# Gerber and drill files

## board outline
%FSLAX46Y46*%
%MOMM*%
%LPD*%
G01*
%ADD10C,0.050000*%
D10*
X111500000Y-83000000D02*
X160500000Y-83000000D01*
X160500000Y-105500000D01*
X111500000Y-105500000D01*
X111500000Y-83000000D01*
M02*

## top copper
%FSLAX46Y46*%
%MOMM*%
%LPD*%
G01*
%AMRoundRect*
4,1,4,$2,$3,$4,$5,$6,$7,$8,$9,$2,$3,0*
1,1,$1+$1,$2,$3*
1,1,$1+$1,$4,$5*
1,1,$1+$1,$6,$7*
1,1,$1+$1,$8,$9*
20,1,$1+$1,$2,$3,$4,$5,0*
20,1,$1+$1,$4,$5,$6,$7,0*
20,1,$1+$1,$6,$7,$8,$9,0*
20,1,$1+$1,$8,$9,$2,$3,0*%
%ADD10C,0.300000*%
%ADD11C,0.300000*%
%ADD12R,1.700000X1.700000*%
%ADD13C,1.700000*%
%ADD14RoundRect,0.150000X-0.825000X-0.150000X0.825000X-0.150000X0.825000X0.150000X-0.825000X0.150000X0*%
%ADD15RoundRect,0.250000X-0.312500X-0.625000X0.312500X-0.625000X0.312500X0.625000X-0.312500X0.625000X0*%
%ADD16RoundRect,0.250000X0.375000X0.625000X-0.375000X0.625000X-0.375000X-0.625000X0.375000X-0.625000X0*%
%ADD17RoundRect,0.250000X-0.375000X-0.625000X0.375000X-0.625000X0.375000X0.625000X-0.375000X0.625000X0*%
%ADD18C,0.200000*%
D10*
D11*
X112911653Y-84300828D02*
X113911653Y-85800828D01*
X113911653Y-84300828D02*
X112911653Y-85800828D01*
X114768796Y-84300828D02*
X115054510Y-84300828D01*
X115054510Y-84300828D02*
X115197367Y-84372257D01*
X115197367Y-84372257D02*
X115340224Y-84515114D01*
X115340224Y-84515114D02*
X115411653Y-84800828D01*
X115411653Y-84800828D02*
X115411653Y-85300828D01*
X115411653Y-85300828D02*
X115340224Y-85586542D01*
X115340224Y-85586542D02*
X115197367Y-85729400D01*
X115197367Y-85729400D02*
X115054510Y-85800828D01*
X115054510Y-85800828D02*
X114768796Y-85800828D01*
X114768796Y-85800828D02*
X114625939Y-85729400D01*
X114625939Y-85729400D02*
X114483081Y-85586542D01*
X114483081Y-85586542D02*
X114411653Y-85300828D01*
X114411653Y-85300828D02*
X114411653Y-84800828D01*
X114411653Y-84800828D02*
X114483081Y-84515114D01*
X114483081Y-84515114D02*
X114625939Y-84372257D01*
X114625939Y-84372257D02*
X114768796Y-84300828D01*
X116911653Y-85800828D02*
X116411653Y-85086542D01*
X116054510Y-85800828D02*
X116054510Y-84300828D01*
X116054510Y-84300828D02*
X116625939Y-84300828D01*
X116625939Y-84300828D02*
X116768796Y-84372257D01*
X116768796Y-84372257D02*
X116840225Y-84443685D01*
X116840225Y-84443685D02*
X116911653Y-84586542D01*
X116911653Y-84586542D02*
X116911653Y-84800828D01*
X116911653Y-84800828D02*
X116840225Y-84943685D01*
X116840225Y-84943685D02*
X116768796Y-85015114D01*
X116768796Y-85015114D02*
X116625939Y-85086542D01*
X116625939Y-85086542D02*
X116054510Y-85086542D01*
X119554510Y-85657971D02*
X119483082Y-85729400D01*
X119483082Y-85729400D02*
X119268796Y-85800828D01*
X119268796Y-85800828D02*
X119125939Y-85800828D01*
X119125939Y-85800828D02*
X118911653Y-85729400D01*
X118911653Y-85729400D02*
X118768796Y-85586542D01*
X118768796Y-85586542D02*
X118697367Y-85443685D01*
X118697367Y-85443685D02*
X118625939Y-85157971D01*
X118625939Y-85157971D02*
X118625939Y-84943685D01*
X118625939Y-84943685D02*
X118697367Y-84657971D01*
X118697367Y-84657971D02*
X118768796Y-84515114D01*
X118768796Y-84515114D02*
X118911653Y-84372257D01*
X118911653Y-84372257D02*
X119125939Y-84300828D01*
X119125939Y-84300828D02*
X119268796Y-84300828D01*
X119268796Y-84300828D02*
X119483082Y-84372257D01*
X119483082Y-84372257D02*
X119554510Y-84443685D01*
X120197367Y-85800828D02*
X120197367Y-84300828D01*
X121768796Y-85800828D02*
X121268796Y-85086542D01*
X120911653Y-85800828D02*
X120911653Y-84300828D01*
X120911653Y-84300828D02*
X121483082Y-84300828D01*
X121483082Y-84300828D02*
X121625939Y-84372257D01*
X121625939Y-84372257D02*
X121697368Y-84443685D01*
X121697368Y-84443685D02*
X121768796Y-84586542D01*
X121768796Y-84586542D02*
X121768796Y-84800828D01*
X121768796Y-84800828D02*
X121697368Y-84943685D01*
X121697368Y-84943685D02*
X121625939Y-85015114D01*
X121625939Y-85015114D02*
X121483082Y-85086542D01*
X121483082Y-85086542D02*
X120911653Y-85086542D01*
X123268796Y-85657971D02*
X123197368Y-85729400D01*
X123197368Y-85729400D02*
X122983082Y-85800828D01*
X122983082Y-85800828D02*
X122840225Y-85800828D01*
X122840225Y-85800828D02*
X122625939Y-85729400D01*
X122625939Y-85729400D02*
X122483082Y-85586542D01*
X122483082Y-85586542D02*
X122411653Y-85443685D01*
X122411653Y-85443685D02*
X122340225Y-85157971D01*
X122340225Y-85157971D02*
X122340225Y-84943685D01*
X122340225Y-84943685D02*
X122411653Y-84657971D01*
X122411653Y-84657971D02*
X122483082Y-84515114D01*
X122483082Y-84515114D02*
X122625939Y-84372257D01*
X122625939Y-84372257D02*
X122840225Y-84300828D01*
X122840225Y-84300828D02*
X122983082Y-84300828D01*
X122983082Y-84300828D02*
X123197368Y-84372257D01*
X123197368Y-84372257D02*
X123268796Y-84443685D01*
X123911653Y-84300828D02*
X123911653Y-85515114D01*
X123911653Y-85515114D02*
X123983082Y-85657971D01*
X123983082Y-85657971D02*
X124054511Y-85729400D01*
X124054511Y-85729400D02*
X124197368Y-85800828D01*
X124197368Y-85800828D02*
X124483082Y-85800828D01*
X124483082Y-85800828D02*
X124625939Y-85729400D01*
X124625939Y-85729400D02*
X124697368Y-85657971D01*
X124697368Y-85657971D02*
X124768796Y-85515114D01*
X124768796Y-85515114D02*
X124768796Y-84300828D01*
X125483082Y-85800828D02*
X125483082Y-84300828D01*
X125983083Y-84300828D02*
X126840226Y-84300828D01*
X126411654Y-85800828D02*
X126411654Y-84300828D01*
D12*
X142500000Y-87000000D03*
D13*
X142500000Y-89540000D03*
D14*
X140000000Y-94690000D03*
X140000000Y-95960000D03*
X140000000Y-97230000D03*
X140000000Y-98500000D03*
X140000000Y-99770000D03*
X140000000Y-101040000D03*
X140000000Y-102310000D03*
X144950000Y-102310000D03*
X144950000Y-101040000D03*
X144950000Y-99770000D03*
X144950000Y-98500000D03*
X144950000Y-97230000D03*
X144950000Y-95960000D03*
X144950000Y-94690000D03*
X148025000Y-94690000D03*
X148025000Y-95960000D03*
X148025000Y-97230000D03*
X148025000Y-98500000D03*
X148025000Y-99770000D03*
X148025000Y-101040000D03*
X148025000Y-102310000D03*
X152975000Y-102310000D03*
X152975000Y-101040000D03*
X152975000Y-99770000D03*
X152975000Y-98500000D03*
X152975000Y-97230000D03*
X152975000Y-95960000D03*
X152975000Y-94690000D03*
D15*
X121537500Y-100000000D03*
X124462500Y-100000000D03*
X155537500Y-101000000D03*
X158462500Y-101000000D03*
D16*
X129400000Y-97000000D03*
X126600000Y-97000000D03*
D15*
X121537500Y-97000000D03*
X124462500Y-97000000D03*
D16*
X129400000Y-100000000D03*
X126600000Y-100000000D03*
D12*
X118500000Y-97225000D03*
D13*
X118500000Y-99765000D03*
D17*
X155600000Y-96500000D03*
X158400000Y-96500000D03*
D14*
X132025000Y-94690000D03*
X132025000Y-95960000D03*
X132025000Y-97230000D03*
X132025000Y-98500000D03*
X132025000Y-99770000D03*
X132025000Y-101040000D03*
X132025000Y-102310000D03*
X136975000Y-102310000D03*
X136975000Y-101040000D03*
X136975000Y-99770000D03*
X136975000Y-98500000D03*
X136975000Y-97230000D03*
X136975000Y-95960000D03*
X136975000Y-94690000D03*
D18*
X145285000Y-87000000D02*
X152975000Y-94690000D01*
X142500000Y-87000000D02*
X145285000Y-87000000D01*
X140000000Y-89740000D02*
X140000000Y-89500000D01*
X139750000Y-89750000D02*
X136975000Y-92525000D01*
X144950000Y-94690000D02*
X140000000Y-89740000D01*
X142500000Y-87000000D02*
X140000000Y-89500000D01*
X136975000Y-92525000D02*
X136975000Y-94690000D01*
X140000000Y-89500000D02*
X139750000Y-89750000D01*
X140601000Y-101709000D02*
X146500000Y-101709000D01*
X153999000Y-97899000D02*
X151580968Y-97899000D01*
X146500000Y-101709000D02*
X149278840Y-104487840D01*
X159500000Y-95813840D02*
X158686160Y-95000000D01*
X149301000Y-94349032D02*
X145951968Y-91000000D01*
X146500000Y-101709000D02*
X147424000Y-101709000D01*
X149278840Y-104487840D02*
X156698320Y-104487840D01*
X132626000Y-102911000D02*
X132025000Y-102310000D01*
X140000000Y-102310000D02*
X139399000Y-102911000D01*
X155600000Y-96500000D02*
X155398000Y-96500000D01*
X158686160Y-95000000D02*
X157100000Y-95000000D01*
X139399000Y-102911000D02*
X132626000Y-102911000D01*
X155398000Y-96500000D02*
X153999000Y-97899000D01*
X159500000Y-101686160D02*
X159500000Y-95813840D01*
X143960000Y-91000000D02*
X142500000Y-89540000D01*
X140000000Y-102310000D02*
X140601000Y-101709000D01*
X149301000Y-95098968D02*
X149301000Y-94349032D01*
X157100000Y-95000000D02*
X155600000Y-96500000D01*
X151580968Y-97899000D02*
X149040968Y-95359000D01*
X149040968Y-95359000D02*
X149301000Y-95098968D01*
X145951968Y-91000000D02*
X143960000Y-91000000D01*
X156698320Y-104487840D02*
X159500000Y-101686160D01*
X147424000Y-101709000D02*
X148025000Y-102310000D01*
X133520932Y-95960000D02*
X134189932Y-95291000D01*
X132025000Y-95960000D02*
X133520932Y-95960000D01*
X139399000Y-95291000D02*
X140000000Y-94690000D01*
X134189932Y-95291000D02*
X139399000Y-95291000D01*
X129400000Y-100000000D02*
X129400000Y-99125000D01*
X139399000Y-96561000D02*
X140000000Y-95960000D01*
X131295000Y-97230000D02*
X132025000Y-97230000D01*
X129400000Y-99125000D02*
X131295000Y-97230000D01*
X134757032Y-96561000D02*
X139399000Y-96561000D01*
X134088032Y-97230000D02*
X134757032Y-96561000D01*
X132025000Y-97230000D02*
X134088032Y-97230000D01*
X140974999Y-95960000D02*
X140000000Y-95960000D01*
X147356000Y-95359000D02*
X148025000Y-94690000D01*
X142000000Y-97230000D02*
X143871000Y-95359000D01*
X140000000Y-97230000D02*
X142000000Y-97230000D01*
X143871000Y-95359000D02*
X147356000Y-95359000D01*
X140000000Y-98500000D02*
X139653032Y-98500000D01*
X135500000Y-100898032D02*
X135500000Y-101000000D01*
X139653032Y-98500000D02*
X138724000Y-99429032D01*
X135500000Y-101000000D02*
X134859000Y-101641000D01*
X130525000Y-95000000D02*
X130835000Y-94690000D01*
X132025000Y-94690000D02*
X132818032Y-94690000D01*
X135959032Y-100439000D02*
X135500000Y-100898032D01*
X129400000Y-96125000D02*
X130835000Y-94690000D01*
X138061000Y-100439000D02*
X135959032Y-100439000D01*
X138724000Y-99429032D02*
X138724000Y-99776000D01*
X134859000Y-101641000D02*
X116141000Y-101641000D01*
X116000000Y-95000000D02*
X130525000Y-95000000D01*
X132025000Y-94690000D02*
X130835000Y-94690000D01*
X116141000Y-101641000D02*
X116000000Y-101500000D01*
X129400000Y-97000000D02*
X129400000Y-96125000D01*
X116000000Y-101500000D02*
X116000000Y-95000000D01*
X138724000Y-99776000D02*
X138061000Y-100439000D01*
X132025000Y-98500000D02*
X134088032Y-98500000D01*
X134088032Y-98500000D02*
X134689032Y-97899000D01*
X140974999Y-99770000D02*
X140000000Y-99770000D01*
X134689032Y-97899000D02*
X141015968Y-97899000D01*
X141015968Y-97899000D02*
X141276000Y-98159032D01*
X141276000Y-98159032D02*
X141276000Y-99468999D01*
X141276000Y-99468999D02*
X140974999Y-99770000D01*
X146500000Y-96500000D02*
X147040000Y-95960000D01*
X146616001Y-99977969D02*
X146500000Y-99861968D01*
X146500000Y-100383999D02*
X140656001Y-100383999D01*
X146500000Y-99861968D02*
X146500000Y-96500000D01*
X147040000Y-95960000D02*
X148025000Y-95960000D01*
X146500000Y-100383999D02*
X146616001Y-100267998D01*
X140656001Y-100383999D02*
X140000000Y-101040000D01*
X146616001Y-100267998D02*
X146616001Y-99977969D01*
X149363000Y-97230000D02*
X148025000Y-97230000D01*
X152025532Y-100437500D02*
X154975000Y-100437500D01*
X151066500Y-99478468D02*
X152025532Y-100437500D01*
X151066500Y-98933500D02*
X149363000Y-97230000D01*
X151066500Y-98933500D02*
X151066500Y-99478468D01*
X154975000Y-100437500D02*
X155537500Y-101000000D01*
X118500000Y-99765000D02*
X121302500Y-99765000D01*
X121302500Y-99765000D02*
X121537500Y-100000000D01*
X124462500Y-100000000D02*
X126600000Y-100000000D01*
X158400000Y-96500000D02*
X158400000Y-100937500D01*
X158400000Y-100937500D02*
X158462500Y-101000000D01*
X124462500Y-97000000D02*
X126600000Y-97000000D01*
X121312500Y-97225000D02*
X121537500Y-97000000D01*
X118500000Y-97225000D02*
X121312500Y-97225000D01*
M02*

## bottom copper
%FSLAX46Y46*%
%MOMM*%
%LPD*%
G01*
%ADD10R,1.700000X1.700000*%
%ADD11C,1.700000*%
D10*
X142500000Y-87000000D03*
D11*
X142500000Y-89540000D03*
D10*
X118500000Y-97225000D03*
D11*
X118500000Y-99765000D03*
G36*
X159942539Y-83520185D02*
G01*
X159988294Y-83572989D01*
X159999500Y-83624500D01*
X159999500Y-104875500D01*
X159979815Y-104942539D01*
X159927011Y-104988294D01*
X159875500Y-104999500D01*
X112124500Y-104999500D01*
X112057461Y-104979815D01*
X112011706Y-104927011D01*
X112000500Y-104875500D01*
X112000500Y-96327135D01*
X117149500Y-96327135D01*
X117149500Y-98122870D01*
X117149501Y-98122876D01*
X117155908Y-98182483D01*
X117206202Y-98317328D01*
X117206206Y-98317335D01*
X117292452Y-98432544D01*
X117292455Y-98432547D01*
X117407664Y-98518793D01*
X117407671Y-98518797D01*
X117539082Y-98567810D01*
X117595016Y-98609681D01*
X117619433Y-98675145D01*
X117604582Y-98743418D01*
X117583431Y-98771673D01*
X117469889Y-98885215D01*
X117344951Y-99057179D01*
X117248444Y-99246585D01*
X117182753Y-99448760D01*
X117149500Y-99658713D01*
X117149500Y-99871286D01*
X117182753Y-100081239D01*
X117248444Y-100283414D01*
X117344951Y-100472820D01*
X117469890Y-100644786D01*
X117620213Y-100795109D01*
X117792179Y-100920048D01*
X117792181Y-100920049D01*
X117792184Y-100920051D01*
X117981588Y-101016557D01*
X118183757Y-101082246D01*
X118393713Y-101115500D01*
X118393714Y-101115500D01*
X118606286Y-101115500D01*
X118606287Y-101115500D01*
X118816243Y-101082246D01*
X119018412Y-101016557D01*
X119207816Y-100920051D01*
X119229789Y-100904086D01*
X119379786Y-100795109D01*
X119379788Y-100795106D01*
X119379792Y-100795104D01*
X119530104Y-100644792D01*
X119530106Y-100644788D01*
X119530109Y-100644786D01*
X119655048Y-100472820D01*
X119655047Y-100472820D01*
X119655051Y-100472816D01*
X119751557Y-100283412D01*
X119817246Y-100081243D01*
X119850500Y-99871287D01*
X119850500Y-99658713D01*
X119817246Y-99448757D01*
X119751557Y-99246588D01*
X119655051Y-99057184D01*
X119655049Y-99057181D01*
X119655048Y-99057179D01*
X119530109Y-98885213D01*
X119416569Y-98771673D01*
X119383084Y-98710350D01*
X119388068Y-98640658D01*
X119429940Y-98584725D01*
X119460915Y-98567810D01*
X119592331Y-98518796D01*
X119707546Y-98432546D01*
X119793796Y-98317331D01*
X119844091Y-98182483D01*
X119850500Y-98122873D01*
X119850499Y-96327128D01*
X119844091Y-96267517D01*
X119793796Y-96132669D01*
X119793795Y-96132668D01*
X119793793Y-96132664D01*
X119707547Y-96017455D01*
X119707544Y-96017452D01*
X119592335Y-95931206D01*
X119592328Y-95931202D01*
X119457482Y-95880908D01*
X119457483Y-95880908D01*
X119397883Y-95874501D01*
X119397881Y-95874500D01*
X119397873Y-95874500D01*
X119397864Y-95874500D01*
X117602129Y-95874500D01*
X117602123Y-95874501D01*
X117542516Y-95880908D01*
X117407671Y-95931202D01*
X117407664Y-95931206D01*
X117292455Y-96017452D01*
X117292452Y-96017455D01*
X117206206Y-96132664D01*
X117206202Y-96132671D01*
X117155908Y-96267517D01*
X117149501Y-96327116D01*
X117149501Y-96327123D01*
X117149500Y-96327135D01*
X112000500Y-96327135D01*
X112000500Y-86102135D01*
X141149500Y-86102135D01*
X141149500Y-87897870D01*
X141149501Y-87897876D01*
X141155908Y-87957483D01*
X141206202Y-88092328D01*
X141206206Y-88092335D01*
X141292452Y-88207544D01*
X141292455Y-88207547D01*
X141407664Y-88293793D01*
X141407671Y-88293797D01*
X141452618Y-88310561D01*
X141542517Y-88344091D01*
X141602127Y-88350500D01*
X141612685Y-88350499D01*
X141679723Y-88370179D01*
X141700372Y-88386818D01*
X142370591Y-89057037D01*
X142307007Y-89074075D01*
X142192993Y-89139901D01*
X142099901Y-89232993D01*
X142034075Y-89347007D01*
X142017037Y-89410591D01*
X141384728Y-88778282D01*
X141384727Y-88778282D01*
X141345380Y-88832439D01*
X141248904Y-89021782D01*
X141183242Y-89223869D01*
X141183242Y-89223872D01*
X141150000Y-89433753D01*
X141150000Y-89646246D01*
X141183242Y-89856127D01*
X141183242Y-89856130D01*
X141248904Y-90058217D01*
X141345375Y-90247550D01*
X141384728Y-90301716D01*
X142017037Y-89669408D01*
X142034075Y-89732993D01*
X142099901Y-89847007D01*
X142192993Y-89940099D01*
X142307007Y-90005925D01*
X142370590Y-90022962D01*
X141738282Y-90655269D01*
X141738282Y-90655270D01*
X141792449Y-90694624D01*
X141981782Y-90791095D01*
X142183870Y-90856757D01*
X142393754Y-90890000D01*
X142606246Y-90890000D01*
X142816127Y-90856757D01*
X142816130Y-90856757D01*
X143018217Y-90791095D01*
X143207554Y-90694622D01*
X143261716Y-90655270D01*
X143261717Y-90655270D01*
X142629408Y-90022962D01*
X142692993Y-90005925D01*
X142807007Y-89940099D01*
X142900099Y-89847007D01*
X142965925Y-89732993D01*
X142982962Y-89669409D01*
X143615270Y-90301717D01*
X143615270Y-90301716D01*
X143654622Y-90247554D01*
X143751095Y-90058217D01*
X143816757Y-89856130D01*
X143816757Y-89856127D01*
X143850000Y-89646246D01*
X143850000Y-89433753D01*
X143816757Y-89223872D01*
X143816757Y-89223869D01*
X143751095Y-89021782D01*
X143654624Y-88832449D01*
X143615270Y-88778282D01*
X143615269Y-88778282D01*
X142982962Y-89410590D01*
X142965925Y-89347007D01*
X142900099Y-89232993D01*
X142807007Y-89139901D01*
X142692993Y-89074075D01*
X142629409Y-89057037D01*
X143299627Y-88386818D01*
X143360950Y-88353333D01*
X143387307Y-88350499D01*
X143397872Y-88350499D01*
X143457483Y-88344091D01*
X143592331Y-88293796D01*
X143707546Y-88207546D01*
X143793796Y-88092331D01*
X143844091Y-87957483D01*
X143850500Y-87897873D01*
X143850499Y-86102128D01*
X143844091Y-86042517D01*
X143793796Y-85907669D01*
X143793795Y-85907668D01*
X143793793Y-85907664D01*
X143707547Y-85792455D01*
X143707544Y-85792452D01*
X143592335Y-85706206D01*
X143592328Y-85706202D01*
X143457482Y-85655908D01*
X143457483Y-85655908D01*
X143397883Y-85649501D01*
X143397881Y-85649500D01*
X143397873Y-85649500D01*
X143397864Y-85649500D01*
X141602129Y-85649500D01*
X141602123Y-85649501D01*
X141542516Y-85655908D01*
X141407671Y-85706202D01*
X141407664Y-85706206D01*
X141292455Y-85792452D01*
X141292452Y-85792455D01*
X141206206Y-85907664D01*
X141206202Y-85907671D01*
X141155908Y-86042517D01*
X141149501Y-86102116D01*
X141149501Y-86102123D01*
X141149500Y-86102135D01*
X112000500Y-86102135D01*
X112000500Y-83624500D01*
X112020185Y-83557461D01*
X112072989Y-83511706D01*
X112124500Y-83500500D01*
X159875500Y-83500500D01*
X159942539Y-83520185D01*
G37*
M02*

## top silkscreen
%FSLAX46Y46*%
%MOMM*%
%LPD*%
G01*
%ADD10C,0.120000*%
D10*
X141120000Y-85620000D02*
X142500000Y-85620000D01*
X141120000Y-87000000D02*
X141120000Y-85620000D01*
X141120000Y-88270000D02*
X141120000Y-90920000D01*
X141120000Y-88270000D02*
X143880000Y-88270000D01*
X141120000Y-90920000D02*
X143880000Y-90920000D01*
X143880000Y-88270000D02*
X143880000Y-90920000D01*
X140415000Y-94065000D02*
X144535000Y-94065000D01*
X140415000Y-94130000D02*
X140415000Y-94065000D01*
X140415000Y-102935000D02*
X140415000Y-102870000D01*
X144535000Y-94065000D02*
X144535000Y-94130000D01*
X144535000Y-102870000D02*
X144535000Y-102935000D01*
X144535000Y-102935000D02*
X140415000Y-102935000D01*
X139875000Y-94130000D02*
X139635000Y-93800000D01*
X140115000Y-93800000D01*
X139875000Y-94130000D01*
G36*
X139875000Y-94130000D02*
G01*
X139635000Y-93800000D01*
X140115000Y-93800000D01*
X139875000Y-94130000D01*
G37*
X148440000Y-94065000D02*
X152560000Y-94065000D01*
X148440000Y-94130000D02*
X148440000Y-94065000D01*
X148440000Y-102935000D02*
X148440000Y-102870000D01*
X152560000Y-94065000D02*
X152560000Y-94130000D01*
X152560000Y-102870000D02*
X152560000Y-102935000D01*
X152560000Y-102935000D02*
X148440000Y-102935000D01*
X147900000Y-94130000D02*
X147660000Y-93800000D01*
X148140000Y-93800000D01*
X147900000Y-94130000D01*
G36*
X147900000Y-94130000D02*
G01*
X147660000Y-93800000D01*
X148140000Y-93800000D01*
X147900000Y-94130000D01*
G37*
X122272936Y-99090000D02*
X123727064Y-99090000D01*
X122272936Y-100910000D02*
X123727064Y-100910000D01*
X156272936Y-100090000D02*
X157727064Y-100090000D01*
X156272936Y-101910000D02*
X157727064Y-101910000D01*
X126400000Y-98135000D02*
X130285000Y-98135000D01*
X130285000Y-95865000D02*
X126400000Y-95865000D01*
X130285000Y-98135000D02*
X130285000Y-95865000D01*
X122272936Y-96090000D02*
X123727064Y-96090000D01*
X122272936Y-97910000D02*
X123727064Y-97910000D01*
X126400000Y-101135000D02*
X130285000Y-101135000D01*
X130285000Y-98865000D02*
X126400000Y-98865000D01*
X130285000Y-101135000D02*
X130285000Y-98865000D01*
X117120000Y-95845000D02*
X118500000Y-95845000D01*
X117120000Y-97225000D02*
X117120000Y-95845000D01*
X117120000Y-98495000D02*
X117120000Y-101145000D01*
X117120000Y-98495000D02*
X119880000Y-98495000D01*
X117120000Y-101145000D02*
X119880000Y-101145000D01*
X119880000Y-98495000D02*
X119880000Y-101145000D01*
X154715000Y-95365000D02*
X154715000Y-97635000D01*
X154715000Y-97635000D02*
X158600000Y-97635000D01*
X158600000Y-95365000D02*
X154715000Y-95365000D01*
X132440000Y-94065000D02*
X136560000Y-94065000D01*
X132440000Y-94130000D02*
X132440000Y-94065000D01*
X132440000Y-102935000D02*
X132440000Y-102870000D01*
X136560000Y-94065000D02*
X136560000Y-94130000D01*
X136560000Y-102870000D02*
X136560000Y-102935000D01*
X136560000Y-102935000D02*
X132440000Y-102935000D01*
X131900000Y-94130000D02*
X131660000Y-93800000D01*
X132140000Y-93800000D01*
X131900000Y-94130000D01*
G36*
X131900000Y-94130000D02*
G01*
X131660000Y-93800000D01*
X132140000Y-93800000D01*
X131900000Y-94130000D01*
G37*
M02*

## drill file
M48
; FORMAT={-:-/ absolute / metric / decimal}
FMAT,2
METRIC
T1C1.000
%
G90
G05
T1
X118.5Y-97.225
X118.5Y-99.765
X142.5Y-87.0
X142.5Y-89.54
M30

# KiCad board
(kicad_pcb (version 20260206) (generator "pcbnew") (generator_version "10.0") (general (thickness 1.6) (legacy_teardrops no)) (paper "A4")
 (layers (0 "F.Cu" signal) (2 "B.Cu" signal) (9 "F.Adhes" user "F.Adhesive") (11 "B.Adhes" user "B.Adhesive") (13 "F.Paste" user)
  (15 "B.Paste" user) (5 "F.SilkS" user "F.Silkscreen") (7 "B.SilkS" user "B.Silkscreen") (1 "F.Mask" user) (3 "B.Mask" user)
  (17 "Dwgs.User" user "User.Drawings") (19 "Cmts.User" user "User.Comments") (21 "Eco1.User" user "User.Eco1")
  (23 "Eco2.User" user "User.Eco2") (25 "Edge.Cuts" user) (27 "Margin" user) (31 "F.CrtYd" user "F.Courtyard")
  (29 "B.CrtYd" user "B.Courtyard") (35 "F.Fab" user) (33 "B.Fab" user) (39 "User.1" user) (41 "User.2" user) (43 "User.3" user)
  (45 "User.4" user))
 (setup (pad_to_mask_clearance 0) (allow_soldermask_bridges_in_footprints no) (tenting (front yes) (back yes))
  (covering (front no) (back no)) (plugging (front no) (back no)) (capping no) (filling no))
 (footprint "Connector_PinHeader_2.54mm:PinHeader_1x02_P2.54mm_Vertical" (layer "F.Cu") (at 142.5 87)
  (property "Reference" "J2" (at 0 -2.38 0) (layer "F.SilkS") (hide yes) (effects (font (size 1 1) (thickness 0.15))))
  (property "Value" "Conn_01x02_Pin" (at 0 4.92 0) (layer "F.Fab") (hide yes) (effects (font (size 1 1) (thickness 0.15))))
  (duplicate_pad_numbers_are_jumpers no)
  (fp_line (start -1.38 -1.38) (end 0 -1.38) (stroke (width 0.12) (type solid)) (layer "F.SilkS"))
  (fp_line (start -1.38 0) (end -1.38 -1.38) (stroke (width 0.12) (type solid)) (layer "F.SilkS"))
  (fp_line (start -1.38 1.27) (end -1.38 3.92) (stroke (width 0.12) (type solid)) (layer "F.SilkS"))
  (fp_line (start -1.38 1.27) (end 1.38 1.27) (stroke (width 0.12) (type solid)) (layer "F.SilkS"))
  (fp_line (start -1.38 3.92) (end 1.38 3.92) (stroke (width 0.12) (type solid)) (layer "F.SilkS"))
  (fp_line (start 1.38 1.27) (end 1.38 3.92) (stroke (width 0.12) (type solid)) (layer "F.SilkS"))
  (pad "1" thru_hole rect (at 0 0) (size 1.7 1.7) (drill 1) (layers "*.Cu" "*.Mask") (remove_unused_layers no) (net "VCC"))
  (pad "2" thru_hole circle (at 0 2.54) (size 1.7 1.7) (drill 1) (layers "*.Cu" "*.Mask") (remove_unused_layers no) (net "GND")))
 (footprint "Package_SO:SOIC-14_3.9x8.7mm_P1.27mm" (layer "F.Cu") (at 142.475 98.5)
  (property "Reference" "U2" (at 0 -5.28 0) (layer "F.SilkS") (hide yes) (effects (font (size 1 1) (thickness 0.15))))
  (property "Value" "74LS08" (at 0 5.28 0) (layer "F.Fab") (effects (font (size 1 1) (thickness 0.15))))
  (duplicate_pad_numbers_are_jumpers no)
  (fp_line (start -2.06 -4.435) (end 2.06 -4.435) (stroke (width 0.12) (type solid)) (layer "F.SilkS"))
  (fp_line (start -2.06 -4.37) (end -2.06 -4.435) (stroke (width 0.12) (type solid)) (layer "F.SilkS"))
  (fp_line (start -2.06 4.435) (end -2.06 4.37) (stroke (width 0.12) (type solid)) (layer "F.SilkS"))
  (fp_line (start 2.06 -4.435) (end 2.06 -4.37) (stroke (width 0.12) (type solid)) (layer "F.SilkS"))
  (fp_line (start 2.06 4.37) (end 2.06 4.435) (stroke (width 0.12) (type solid)) (layer "F.SilkS"))
  (fp_line (start 2.06 4.435) (end -2.06 4.435) (stroke (width 0.12) (type solid)) (layer "F.SilkS"))
  (fp_poly (pts (xy -2.6 -4.37) (xy -2.84 -4.7) (xy -2.36 -4.7)) (stroke (width 0.12) (type solid)) (fill yes) (layer "F.SilkS"))
  (pad "1" smd roundrect (at -2.475 -3.81) (size 1.95 0.6) (layers "F.Cu" "F.Mask" "F.Paste") (roundrect_rratio 0.25) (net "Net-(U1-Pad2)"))
  (pad "2" smd roundrect (at -2.475 -2.54) (size 1.95 0.6) (layers "F.Cu" "F.Mask" "F.Paste") (roundrect_rratio 0.25) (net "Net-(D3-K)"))
  (pad "3" smd roundrect (at -2.475 -1.27) (size 1.95 0.6) (layers "F.Cu" "F.Mask" "F.Paste") (roundrect_rratio 0.25) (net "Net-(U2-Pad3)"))
  (pad "4" smd roundrect (at -2.475 0) (size 1.95 0.6) (layers "F.Cu" "F.Mask" "F.Paste") (roundrect_rratio 0.25) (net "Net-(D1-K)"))
  (pad "5" smd roundrect (at -2.475 1.27) (size 1.95 0.6) (layers "F.Cu" "F.Mask" "F.Paste") (roundrect_rratio 0.25) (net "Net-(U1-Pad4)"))
  (pad "6" smd roundrect (at -2.475 2.54) (size 1.95 0.6) (layers "F.Cu" "F.Mask" "F.Paste") (roundrect_rratio 0.25) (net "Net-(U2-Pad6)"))
  (pad "7" smd roundrect (at -2.475 3.81) (size 1.95 0.6) (layers "F.Cu" "F.Mask" "F.Paste") (roundrect_rratio 0.25) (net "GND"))
  (pad "8" smd roundrect (at 2.475 3.81) (size 1.95 0.6) (layers "F.Cu" "F.Mask" "F.Paste") (roundrect_rratio 0.25))
  (pad "9" smd roundrect (at 2.475 2.54) (size 1.95 0.6) (layers "F.Cu" "F.Mask" "F.Paste") (roundrect_rratio 0.25))
  (pad "10" smd roundrect (at 2.475 1.27) (size 1.95 0.6) (layers "F.Cu" "F.Mask" "F.Paste") (roundrect_rratio 0.25))
  (pad "11" smd roundrect (at 2.475 0) (size 1.95 0.6) (layers "F.Cu" "F.Mask" "F.Paste") (roundrect_rratio 0.25))
  (pad "12" smd roundrect (at 2.475 -1.27) (size 1.95 0.6) (layers "F.Cu" "F.Mask" "F.Paste") (roundrect_rratio 0.25))
  (pad "13" smd roundrect (at 2.475 -2.54) (size 1.95 0.6) (layers "F.Cu" "F.Mask" "F.Paste") (roundrect_rratio 0.25))
  (pad "14" smd roundrect (at 2.475 -3.81) (size 1.95 0.6) (layers "F.Cu" "F.Mask" "F.Paste") (roundrect_rratio 0.25) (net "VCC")))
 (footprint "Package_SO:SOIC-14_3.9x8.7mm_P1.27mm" (layer "F.Cu") (at 150.5 98.5)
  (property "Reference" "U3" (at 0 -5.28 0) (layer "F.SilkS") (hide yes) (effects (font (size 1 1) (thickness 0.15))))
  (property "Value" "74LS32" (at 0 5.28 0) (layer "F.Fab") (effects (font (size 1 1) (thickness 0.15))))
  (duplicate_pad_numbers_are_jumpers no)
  (fp_line (start -2.06 -4.435) (end 2.06 -4.435) (stroke (width 0.12) (type solid)) (layer "F.SilkS"))
  (fp_line (start -2.06 -4.37) (end -2.06 -4.435) (stroke (width 0.12) (type solid)) (layer "F.SilkS"))
  (fp_line (start -2.06 4.435) (end -2.06 4.37) (stroke (width 0.12) (type solid)) (layer "F.SilkS"))
  (fp_line (start 2.06 -4.435) (end 2.06 -4.37) (stroke (width 0.12) (type solid)) (layer "F.SilkS"))
  (fp_line (start 2.06 4.37) (end 2.06 4.435) (stroke (width 0.12) (type solid)) (layer "F.SilkS"))
  (fp_line (start 2.06 4.435) (end -2.06 4.435) (stroke (width 0.12) (type solid)) (layer "F.SilkS"))
  (fp_poly (pts (xy -2.6 -4.37) (xy -2.84 -4.7) (xy -2.36 -4.7)) (stroke (width 0.12) (type solid)) (fill yes) (layer "F.SilkS"))
  (pad "1" smd roundrect (at -2.475 -3.81) (size 1.95 0.6) (layers "F.Cu" "F.Mask" "F.Paste") (roundrect_rratio 0.25) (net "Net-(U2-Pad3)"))
  (pad "2" smd roundrect (at -2.475 -2.54) (size 1.95 0.6) (layers "F.Cu" "F.Mask" "F.Paste") (roundrect_rratio 0.25) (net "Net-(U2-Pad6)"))
  (pad "3" smd roundrect (at -2.475 -1.27) (size 1.95 0.6) (layers "F.Cu" "F.Mask" "F.Paste") (roundrect_rratio 0.25) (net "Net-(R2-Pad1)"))
  (pad "4" smd roundrect (at -2.475 0) (size 1.95 0.6) (layers "F.Cu" "F.Mask" "F.Paste") (roundrect_rratio 0.25))
  (pad "5" smd roundrect (at -2.475 1.27) (size 1.95 0.6) (layers "F.Cu" "F.Mask" "F.Paste") (roundrect_rratio 0.25))
  (pad "6" smd roundrect (at -2.475 2.54) (size 1.95 0.6) (layers "F.Cu" "F.Mask" "F.Paste") (roundrect_rratio 0.25))
  (pad "7" smd roundrect (at -2.475 3.81) (size 1.95 0.6) (layers "F.Cu" "F.Mask" "F.Paste") (roundrect_rratio 0.25) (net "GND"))
  (pad "8" smd roundrect (at 2.475 3.81) (size 1.95 0.6) (layers "F.Cu" "F.Mask" "F.Paste") (roundrect_rratio 0.25))
  (pad "9" smd roundrect (at 2.475 2.54) (size 1.95 0.6) (layers "F.Cu" "F.Mask" "F.Paste") (roundrect_rratio 0.25))
  (pad "10" smd roundrect (at 2.475 1.27) (size 1.95 0.6) (layers "F.Cu" "F.Mask" "F.Paste") (roundrect_rratio 0.25))
  (pad "11" smd roundrect (at 2.475 0) (size 1.95 0.6) (layers "F.Cu" "F.Mask" "F.Paste") (roundrect_rratio 0.25))
  (pad "12" smd roundrect (at 2.475 -1.27) (size 1.95 0.6) (layers "F.Cu" "F.Mask" "F.Paste") (roundrect_rratio 0.25))
  (pad "13" smd roundrect (at 2.475 -2.54) (size 1.95 0.6) (layers "F.Cu" "F.Mask" "F.Paste") (roundrect_rratio 0.25))
  (pad "14" smd roundrect (at 2.475 -3.81) (size 1.95 0.6) (layers "F.Cu" "F.Mask" "F.Paste") (roundrect_rratio 0.25) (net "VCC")))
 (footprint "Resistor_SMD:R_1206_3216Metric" (layer "F.Cu") (at 123 100)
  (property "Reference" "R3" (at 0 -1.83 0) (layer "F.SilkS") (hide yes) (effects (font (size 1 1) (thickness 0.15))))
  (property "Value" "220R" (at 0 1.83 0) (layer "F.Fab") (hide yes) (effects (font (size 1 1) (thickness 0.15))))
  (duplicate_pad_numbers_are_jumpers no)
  (fp_line (start -0.727064 -0.91) (end 0.727064 -0.91) (stroke (width 0.12) (type solid)) (layer "F.SilkS"))
  (fp_line (start -0.727064 0.91) (end 0.727064 0.91) (stroke (width 0.12) (type solid)) (layer "F.SilkS"))
  (pad "1" smd roundrect (at -1.4625 0) (size 1.125 1.75) (layers "F.Cu" "F.Mask" "F.Paste") (roundrect_rratio 0.222222)
   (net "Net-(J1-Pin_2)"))
  (pad "2" smd roundrect (at 1.4625 0) (size 1.125 1.75) (layers "F.Cu" "F.Mask" "F.Paste") (roundrect_rratio 0.222222) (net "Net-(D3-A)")))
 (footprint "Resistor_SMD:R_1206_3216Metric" (layer "F.Cu") (at 157 101)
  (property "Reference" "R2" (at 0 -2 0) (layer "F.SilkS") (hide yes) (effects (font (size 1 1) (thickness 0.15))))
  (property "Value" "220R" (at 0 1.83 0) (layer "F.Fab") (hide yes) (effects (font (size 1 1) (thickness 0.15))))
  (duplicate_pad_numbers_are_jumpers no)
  (fp_line (start -0.727064 -0.91) (end 0.727064 -0.91) (stroke (width 0.12) (type solid)) (layer "F.SilkS"))
  (fp_line (start -0.727064 0.91) (end 0.727064 0.91) (stroke (width 0.12) (type solid)) (layer "F.SilkS"))
  (pad "1" smd roundrect (at -1.4625 0) (size 1.125 1.75) (layers "F.Cu" "F.Mask" "F.Paste") (roundrect_rratio 0.222222)
   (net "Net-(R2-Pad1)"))
  (pad "2" smd roundrect (at 1.4625 0) (size 1.125 1.75) (layers "F.Cu" "F.Mask" "F.Paste") (roundrect_rratio 0.222222) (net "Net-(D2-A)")))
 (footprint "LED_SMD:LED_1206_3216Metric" (layer "F.Cu") (at 128 97 180)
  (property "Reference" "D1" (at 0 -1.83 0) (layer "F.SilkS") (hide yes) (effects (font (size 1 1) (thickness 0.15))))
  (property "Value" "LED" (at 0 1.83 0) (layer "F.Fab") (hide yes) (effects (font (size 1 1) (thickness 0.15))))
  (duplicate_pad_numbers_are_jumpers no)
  (fp_line (start 1.6 -1.135) (end -2.285 -1.135) (stroke (width 0.12) (type solid)) (layer "F.SilkS"))
  (fp_line (start -2.285 1.135) (end 1.6 1.135) (stroke (width 0.12) (type solid)) (layer "F.SilkS"))
  (fp_line (start -2.285 -1.135) (end -2.285 1.135) (stroke (width 0.12) (type solid)) (layer "F.SilkS"))
  (pad "1" smd roundrect (at -1.4 0 180) (size 1.25 1.75) (layers "F.Cu" "F.Mask" "F.Paste") (roundrect_rratio 0.2) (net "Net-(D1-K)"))
  (pad "2" smd roundrect (at 1.4 0 180) (size 1.25 1.75) (layers "F.Cu" "F.Mask" "F.Paste") (roundrect_rratio 0.2) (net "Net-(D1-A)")))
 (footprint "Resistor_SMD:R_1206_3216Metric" (layer "F.Cu") (at 123 97)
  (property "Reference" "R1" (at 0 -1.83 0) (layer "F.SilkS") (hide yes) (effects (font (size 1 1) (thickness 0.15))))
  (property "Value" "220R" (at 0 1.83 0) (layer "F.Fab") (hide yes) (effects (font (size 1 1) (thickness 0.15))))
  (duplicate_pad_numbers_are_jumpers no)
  (fp_line (start -0.727064 -0.91) (end 0.727064 -0.91) (stroke (width 0.12) (type solid)) (layer "F.SilkS"))
  (fp_line (start -0.727064 0.91) (end 0.727064 0.91) (stroke (width 0.12) (type solid)) (layer "F.SilkS"))
  (pad "1" smd roundrect (at -1.4625 0) (size 1.125 1.75) (layers "F.Cu" "F.Mask" "F.Paste") (roundrect_rratio 0.222222)
   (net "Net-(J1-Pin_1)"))
  (pad "2" smd roundrect (at 1.4625 0) (size 1.125 1.75) (layers "F.Cu" "F.Mask" "F.Paste") (roundrect_rratio 0.222222) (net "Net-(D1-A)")))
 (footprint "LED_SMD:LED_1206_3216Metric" (layer "F.Cu") (at 128 100 180)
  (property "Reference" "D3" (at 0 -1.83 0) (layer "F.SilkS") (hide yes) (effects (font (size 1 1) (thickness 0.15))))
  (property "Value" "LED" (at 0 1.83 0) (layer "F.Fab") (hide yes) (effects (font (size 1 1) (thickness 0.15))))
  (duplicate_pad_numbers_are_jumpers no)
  (fp_line (start 1.6 -1.135) (end -2.285 -1.135) (stroke (width 0.12) (type solid)) (layer "F.SilkS"))
  (fp_line (start -2.285 1.135) (end 1.6 1.135) (stroke (width 0.12) (type solid)) (layer "F.SilkS"))
  (fp_line (start -2.285 -1.135) (end -2.285 1.135) (stroke (width 0.12) (type solid)) (layer "F.SilkS"))
  (pad "1" smd roundrect (at -1.4 0 180) (size 1.25 1.75) (layers "F.Cu" "F.Mask" "F.Paste") (roundrect_rratio 0.2) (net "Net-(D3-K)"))
  (pad "2" smd roundrect (at 1.4 0 180) (size 1.25 1.75) (layers "F.Cu" "F.Mask" "F.Paste") (roundrect_rratio 0.2) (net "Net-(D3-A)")))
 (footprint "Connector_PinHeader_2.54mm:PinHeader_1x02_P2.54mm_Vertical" (layer "F.Cu") (at 118.5 97.225)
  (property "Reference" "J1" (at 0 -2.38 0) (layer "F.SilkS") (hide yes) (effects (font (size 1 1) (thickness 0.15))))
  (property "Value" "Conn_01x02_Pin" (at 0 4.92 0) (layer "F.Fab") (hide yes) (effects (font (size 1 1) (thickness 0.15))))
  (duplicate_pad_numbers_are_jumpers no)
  (fp_line (start -1.38 -1.38) (end 0 -1.38) (stroke (width 0.12) (type solid)) (layer "F.SilkS"))
  (fp_line (start -1.38 0) (end -1.38 -1.38) (stroke (width 0.12) (type solid)) (layer "F.SilkS"))
  (fp_line (start -1.38 1.27) (end -1.38 3.92) (stroke (width 0.12) (type solid)) (layer "F.SilkS"))
  (fp_line (start -1.38 1.27) (end 1.38 1.27) (stroke (width 0.12) (type solid)) (layer "F.SilkS"))
  (fp_line (start -1.38 3.92) (end 1.38 3.92) (stroke (width 0.12) (type solid)) (layer "F.SilkS"))
  (fp_line (start 1.38 1.27) (end 1.38 3.92) (stroke (width 0.12) (type solid)) (layer "F.SilkS"))
  (pad "1" thru_hole rect (at 0 0) (size 1.7 1.7) (drill 1) (layers "*.Cu" "*.Mask") (remove_unused_layers no) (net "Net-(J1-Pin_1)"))
  (pad "2" thru_hole circle (at 0 2.54) (size 1.7 1.7) (drill 1) (layers "*.Cu" "*.Mask") (remove_unused_layers no) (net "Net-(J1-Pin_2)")))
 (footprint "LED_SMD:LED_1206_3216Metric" (layer "F.Cu") (at 157 96.5)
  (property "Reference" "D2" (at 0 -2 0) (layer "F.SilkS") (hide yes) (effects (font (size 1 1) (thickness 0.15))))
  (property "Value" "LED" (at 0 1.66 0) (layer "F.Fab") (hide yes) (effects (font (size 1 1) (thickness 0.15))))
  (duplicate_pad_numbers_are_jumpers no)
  (fp_line (start -2.285 -1.135) (end -2.285 1.135) (stroke (width 0.12) (type solid)) (layer "F.SilkS"))
  (fp_line (start -2.285 1.135) (end 1.6 1.135) (stroke (width 0.12) (type solid)) (layer "F.SilkS"))
  (fp_line (start 1.6 -1.135) (end -2.285 -1.135) (stroke (width 0.12) (type solid)) (layer "F.SilkS"))
  (pad "1" smd roundrect (at -1.4 0) (size 1.25 1.75) (layers "F.Cu" "F.Mask" "F.Paste") (roundrect_rratio 0.2) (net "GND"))
  (pad "2" smd roundrect (at 1.4 0) (size 1.25 1.75) (layers "F.Cu" "F.Mask" "F.Paste") (roundrect_rratio 0.2) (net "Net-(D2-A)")))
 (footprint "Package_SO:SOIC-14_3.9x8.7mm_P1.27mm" (layer "F.Cu") (at 134.5 98.5)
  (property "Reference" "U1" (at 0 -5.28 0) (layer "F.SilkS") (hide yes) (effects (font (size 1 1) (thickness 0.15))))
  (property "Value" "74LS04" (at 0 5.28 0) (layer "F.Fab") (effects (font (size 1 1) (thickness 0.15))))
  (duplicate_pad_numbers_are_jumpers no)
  (fp_line (start -2.06 -4.435) (end 2.06 -4.435) (stroke (width 0.12) (type solid)) (layer "F.SilkS"))
  (fp_line (start -2.06 -4.37) (end -2.06 -4.435) (stroke (width 0.12) (type solid)) (layer "F.SilkS"))
  (fp_line (start -2.06 4.435) (end -2.06 4.37) (stroke (width 0.12) (type solid)) (layer "F.SilkS"))
  (fp_line (start 2.06 -4.435) (end 2.06 -4.37) (stroke (width 0.12) (type solid)) (layer "F.SilkS"))
  (fp_line (start 2.06 4.37) (end 2.06 4.435) (stroke (width 0.12) (type solid)) (layer "F.SilkS"))
  (fp_line (start 2.06 4.435) (end -2.06 4.435) (stroke (width 0.12) (type solid)) (layer "F.SilkS"))
  (fp_poly (pts (xy -2.6 -4.37) (xy -2.84 -4.7) (xy -2.36 -4.7)) (stroke (width 0.12) (type solid)) (fill yes) (layer "F.SilkS"))
  (pad "1" smd roundrect (at -2.475 -3.81) (size 1.95 0.6) (layers "F.Cu" "F.Mask" "F.Paste") (roundrect_rratio 0.25) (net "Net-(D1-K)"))
  (pad "2" smd roundrect (at -2.475 -2.54) (size 1.95 0.6) (layers "F.Cu" "F.Mask" "F.Paste") (roundrect_rratio 0.25) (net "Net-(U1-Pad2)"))
  (pad "3" smd roundrect (at -2.475 -1.27) (size 1.95 0.6) (layers "F.Cu" "F.Mask" "F.Paste") (roundrect_rratio 0.25) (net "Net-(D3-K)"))
  (pad "4" smd roundrect (at -2.475 0) (size 1.95 0.6) (layers "F.Cu" "F.Mask" "F.Paste") (roundrect_rratio 0.25) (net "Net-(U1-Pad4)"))
  (pad "5" smd roundrect (at -2.475 1.27) (size 1.95 0.6) (layers "F.Cu" "F.Mask" "F.Paste") (roundrect_rratio 0.25))
  (pad "6" smd roundrect (at -2.475 2.54) (size 1.95 0.6) (layers "F.Cu" "F.Mask" "F.Paste") (roundrect_rratio 0.25))
  (pad "7" smd roundrect (at -2.475 3.81) (size 1.95 0.6) (layers "F.Cu" "F.Mask" "F.Paste") (roundrect_rratio 0.25) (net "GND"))
  (pad "8" smd roundrect (at 2.475 3.81) (size 1.95 0.6) (layers "F.Cu" "F.Mask" "F.Paste") (roundrect_rratio 0.25))
  (pad "9" smd roundrect (at 2.475 2.54) (size 1.95 0.6) (layers "F.Cu" "F.Mask" "F.Paste") (roundrect_rratio 0.25))
  (pad "10" smd roundrect (at 2.475 1.27) (size 1.95 0.6) (layers "F.Cu" "F.Mask" "F.Paste") (roundrect_rratio 0.25))
  (pad "11" smd roundrect (at 2.475 0) (size 1.95 0.6) (layers "F.Cu" "F.Mask" "F.Paste") (roundrect_rratio 0.25))
  (pad "12" smd roundrect (at 2.475 -1.27) (size 1.95 0.6) (layers "F.Cu" "F.Mask" "F.Paste") (roundrect_rratio 0.25))
  (pad "13" smd roundrect (at 2.475 -2.54) (size 1.95 0.6) (layers "F.Cu" "F.Mask" "F.Paste") (roundrect_rratio 0.25))
  (pad "14" smd roundrect (at 2.475 -3.81) (size 1.95 0.6) (layers "F.Cu" "F.Mask" "F.Paste") (roundrect_rratio 0.25) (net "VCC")))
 (gr_rect (start 111.5 83) (end 160.5 105.5) (stroke (width 0.05) (type default)) (fill no) (layer "Edge.Cuts"))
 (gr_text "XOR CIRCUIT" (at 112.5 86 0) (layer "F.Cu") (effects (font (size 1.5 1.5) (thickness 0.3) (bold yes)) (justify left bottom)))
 (segment (start 145.285 87) (end 152.975 94.69) (width 0.2) (layer "F.Cu") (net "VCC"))
 (segment (start 142.5 87) (end 145.285 87) (width 0.2) (layer "F.Cu") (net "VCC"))
 (segment (start 140 89.74) (end 140 89.5) (width 0.2) (layer "F.Cu") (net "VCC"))
 (segment (start 139.75 89.75) (end 136.975 92.525) (width 0.2) (layer "F.Cu") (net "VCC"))
 (segment (start 144.95 94.69) (end 140 89.74) (width 0.2) (layer "F.Cu") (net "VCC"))
 (segment (start 142.5 87) (end 140 89.5) (width 0.2) (layer "F.Cu") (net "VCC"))
 (segment (start 136.975 92.525) (end 136.975 94.69) (width 0.2) (layer "F.Cu") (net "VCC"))
 (segment (start 140 89.5) (end 139.75 89.75) (width 0.2) (layer "F.Cu") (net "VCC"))
 (segment (start 140.601 101.709) (end 146.5 101.709) (width 0.2) (layer "F.Cu") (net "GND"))
 (segment (start 153.999 97.899) (end 151.580968 97.899) (width 0.2) (layer "F.Cu") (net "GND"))
 (segment (start 146.5 101.709) (end 149.27884 104.48784) (width 0.2) (layer "F.Cu") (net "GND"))
 (segment (start 159.5 95.81384) (end 158.68616 95) (width 0.2) (layer "F.Cu") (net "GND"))
 (segment (start 149.301 94.349032) (end 145.951968 91) (width 0.2) (layer "F.Cu") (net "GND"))
 (segment (start 146.5 101.709) (end 147.424 101.709) (width 0.2) (layer "F.Cu") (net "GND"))
 (segment (start 149.27884 104.48784) (end 156.69832 104.48784) (width 0.2) (layer "F.Cu") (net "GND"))
 (segment (start 132.626 102.911) (end 132.025 102.31) (width 0.2) (layer "F.Cu") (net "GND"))
 (segment (start 140 102.31) (end 139.399 102.911) (width 0.2) (layer "F.Cu") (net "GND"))
 (segment (start 155.6 96.5) (end 155.398 96.5) (width 0.2) (layer "F.Cu") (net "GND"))
 (segment (start 158.68616 95) (end 157.1 95) (width 0.2) (layer "F.Cu") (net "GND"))
 (segment (start 139.399 102.911) (end 132.626 102.911) (width 0.2) (layer "F.Cu") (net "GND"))
 (segment (start 155.398 96.5) (end 153.999 97.899) (width 0.2) (layer "F.Cu") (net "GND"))
 (segment (start 159.5 101.68616) (end 159.5 95.81384) (width 0.2) (layer "F.Cu") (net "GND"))
 (segment (start 143.96 91) (end 142.5 89.54) (width 0.2) (layer "F.Cu") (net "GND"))
 (segment (start 140 102.31) (end 140.601 101.709) (width 0.2) (layer "F.Cu") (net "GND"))
 (segment (start 149.301 95.098968) (end 149.301 94.349032) (width 0.2) (layer "F.Cu") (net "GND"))
 (segment (start 157.1 95) (end 155.6 96.5) (width 0.2) (layer "F.Cu") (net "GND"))
 (segment (start 151.580968 97.899) (end 149.040968 95.359) (width 0.2) (layer "F.Cu") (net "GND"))
 (segment (start 149.040968 95.359) (end 149.301 95.098968) (width 0.2) (layer "F.Cu") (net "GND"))
 (segment (start 145.951968 91) (end 143.96 91) (width 0.2) (layer "F.Cu") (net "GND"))
 (segment (start 156.69832 104.48784) (end 159.5 101.68616) (width 0.2) (layer "F.Cu") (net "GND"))
 (segment (start 147.424 101.709) (end 148.025 102.31) (width 0.2) (layer "F.Cu") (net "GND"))
 (segment (start 133.520932 95.96) (end 134.189932 95.291) (width 0.2) (layer "F.Cu") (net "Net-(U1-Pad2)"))
 (segment (start 132.025 95.96) (end 133.520932 95.96) (width 0.2) (layer "F.Cu") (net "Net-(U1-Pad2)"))
 (segment (start 139.399 95.291) (end 140 94.69) (width 0.2) (layer "F.Cu") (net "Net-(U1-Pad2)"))
 (segment (start 134.189932 95.291) (end 139.399 95.291) (width 0.2) (layer "F.Cu") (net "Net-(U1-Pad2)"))
 (segment (start 129.4 100) (end 129.4 99.125) (width 0.2) (layer "F.Cu") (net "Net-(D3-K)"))
 (segment (start 139.399 96.561) (end 140 95.96) (width 0.2) (layer "F.Cu") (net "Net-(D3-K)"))
 (segment (start 131.295 97.23) (end 132.025 97.23) (width 0.2) (layer "F.Cu") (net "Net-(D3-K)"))
 (segment (start 129.4 99.125) (end 131.295 97.23) (width 0.2) (layer "F.Cu") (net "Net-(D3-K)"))
 (segment (start 134.757032 96.561) (end 139.399 96.561) (width 0.2) (layer "F.Cu") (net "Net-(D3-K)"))
 (segment (start 134.088032 97.23) (end 134.757032 96.561) (width 0.2) (layer "F.Cu") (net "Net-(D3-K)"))
 (segment (start 132.025 97.23) (end 134.088032 97.23) (width 0.2) (layer "F.Cu") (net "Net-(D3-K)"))
 (segment (start 140.974999 95.96) (end 140 95.96) (width 0.2) (layer "F.Cu") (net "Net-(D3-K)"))
 (segment (start 147.356 95.359) (end 148.025 94.69) (width 0.2) (layer "F.Cu") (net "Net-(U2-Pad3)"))
 (segment (start 142 97.23) (end 143.871 95.359) (width 0.2) (layer "F.Cu") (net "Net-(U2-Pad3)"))
 (segment (start 140 97.23) (end 142 97.23) (width 0.2) (layer "F.Cu") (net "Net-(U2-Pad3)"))
 (segment (start 143.871 95.359) (end 147.356 95.359) (width 0.2) (layer "F.Cu") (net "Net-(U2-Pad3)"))
 (segment (start 140 98.5) (end 139.653032 98.5) (width 0.2) (layer "F.Cu") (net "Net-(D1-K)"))
 (segment (start 135.5 100.898032) (end 135.5 101) (width 0.2) (layer "F.Cu") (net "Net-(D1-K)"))
 (segment (start 139.653032 98.5) (end 138.724 99.429032) (width 0.2) (layer "F.Cu") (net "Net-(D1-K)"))
 (segment (start 135.5 101) (end 134.859 101.641) (width 0.2) (layer "F.Cu") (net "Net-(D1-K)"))
 (segment (start 130.525 95) (end 130.835 94.69) (width 0.2) (layer "F.Cu") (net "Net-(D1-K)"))
 (segment (start 132.025 94.69) (end 132.818032 94.69) (width 0.2) (layer "F.Cu") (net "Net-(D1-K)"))
 (segment (start 135.959032 100.439) (end 135.5 100.898032) (width 0.2) (layer "F.Cu") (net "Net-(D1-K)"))
 (segment (start 129.4 96.125) (end 130.835 94.69) (width 0.2) (layer "F.Cu") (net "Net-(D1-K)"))
 (segment (start 138.061 100.439) (end 135.959032 100.439) (width 0.2) (layer "F.Cu") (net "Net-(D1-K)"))
 (segment (start 138.724 99.429032) (end 138.724 99.776) (width 0.2) (layer "F.Cu") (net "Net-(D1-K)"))
 (segment (start 134.859 101.641) (end 116.141 101.641) (width 0.2) (layer "F.Cu") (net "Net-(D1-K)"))
 (segment (start 116 95) (end 130.525 95) (width 0.2) (layer "F.Cu") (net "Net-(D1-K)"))
 (segment (start 132.025 94.69) (end 130.835 94.69) (width 0.2) (layer "F.Cu") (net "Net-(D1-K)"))
 (segment (start 116.141 101.641) (end 116 101.5) (width 0.2) (layer "F.Cu") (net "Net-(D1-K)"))
 (segment (start 129.4 97) (end 129.4 96.125) (width 0.2) (layer "F.Cu") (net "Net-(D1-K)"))
 (segment (start 116 101.5) (end 116 95) (width 0.2) (layer "F.Cu") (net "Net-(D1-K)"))
 (segment (start 138.724 99.776) (end 138.061 100.439) (width 0.2) (layer "F.Cu") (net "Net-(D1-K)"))
 (segment (start 132.025 98.5) (end 134.088032 98.5) (width 0.2) (layer "F.Cu") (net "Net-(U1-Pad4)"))
 (segment (start 134.088032 98.5) (end 134.689032 97.899) (width 0.2) (layer "F.Cu") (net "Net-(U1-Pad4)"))
 (segment (start 140.974999 99.77) (end 140 99.77) (width 0.2) (layer "F.Cu") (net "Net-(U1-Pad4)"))
 (segment (start 134.689032 97.899) (end 141.015968 97.899) (width 0.2) (layer "F.Cu") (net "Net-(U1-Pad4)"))
 (segment (start 141.015968 97.899) (end 141.276 98.159032) (width 0.2) (layer "F.Cu") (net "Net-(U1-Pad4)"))
 (segment (start 141.276 98.159032) (end 141.276 99.468999) (width 0.2) (layer "F.Cu") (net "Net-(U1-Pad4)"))
 (segment (start 141.276 99.468999) (end 140.974999 99.77) (width 0.2) (layer "F.Cu") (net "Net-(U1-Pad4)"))
 (segment (start 146.5 96.5) (end 147.04 95.96) (width 0.2) (layer "F.Cu") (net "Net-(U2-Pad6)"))
 (segment (start 146.616001 99.977969) (end 146.5 99.861968) (width 0.2) (layer "F.Cu") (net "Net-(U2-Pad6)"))
 (segment (start 146.5 100.383999) (end 140.656001 100.383999) (width 0.2) (layer "F.Cu") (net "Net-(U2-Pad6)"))
 (segment (start 146.5 99.861968) (end 146.5 96.5) (width 0.2) (layer "F.Cu") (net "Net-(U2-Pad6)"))
 (segment (start 147.04 95.96) (end 148.025 95.96) (width 0.2) (layer "F.Cu") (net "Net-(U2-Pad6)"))
 (segment (start 146.5 100.383999) (end 146.616001 100.267998) (width 0.2) (layer "F.Cu") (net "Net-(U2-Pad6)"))
 (segment (start 140.656001 100.383999) (end 140 101.04) (width 0.2) (layer "F.Cu") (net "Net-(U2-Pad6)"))
 (segment (start 146.616001 100.267998) (end 146.616001 99.977969) (width 0.2) (layer "F.Cu") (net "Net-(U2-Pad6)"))
 (segment (start 149.363 97.23) (end 148.025 97.23) (width 0.2) (layer "F.Cu") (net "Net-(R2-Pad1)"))
 (segment (start 152.025532 100.4375) (end 154.975 100.4375) (width 0.2) (layer "F.Cu") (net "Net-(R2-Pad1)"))
 (segment (start 151.0665 99.478468) (end 152.025532 100.4375) (width 0.2) (layer "F.Cu") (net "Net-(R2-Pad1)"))
 (segment (start 151.0665 98.9335) (end 149.363 97.23) (width 0.2) (layer "F.Cu") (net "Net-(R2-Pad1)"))
 (segment (start 151.0665 98.9335) (end 151.0665 99.478468) (width 0.2) (layer "F.Cu") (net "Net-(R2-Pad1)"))
 (segment (start 154.975 100.4375) (end 155.5375 101) (width 0.2) (layer "F.Cu") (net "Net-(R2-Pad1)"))
 (segment (start 118.5 99.765) (end 121.3025 99.765) (width 0.2) (layer "F.Cu") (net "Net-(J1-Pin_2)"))
 (segment (start 121.3025 99.765) (end 121.5375 100) (width 0.2) (layer "F.Cu") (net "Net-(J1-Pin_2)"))
 (segment (start 124.4625 100) (end 126.6 100) (width 0.2) (layer "F.Cu") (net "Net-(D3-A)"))
 (segment (start 158.4 96.5) (end 158.4 100.9375) (width 0.2) (layer "F.Cu") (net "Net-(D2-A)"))
 (segment (start 158.4 100.9375) (end 158.4625 101) (width 0.2) (layer "F.Cu") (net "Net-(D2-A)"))
 (segment (start 124.4625 97) (end 126.6 97) (width 0.2) (layer "F.Cu") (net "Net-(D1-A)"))
 (segment (start 121.3125 97.225) (end 121.5375 97) (width 0.2) (layer "F.Cu") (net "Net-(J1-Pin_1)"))
 (segment (start 118.5 97.225) (end 121.3125 97.225) (width 0.2) (layer "F.Cu") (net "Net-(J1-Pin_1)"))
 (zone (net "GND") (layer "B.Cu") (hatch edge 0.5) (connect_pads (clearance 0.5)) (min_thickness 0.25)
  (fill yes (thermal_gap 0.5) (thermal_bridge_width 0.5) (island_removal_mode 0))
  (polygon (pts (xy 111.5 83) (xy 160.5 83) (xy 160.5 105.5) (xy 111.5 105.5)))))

